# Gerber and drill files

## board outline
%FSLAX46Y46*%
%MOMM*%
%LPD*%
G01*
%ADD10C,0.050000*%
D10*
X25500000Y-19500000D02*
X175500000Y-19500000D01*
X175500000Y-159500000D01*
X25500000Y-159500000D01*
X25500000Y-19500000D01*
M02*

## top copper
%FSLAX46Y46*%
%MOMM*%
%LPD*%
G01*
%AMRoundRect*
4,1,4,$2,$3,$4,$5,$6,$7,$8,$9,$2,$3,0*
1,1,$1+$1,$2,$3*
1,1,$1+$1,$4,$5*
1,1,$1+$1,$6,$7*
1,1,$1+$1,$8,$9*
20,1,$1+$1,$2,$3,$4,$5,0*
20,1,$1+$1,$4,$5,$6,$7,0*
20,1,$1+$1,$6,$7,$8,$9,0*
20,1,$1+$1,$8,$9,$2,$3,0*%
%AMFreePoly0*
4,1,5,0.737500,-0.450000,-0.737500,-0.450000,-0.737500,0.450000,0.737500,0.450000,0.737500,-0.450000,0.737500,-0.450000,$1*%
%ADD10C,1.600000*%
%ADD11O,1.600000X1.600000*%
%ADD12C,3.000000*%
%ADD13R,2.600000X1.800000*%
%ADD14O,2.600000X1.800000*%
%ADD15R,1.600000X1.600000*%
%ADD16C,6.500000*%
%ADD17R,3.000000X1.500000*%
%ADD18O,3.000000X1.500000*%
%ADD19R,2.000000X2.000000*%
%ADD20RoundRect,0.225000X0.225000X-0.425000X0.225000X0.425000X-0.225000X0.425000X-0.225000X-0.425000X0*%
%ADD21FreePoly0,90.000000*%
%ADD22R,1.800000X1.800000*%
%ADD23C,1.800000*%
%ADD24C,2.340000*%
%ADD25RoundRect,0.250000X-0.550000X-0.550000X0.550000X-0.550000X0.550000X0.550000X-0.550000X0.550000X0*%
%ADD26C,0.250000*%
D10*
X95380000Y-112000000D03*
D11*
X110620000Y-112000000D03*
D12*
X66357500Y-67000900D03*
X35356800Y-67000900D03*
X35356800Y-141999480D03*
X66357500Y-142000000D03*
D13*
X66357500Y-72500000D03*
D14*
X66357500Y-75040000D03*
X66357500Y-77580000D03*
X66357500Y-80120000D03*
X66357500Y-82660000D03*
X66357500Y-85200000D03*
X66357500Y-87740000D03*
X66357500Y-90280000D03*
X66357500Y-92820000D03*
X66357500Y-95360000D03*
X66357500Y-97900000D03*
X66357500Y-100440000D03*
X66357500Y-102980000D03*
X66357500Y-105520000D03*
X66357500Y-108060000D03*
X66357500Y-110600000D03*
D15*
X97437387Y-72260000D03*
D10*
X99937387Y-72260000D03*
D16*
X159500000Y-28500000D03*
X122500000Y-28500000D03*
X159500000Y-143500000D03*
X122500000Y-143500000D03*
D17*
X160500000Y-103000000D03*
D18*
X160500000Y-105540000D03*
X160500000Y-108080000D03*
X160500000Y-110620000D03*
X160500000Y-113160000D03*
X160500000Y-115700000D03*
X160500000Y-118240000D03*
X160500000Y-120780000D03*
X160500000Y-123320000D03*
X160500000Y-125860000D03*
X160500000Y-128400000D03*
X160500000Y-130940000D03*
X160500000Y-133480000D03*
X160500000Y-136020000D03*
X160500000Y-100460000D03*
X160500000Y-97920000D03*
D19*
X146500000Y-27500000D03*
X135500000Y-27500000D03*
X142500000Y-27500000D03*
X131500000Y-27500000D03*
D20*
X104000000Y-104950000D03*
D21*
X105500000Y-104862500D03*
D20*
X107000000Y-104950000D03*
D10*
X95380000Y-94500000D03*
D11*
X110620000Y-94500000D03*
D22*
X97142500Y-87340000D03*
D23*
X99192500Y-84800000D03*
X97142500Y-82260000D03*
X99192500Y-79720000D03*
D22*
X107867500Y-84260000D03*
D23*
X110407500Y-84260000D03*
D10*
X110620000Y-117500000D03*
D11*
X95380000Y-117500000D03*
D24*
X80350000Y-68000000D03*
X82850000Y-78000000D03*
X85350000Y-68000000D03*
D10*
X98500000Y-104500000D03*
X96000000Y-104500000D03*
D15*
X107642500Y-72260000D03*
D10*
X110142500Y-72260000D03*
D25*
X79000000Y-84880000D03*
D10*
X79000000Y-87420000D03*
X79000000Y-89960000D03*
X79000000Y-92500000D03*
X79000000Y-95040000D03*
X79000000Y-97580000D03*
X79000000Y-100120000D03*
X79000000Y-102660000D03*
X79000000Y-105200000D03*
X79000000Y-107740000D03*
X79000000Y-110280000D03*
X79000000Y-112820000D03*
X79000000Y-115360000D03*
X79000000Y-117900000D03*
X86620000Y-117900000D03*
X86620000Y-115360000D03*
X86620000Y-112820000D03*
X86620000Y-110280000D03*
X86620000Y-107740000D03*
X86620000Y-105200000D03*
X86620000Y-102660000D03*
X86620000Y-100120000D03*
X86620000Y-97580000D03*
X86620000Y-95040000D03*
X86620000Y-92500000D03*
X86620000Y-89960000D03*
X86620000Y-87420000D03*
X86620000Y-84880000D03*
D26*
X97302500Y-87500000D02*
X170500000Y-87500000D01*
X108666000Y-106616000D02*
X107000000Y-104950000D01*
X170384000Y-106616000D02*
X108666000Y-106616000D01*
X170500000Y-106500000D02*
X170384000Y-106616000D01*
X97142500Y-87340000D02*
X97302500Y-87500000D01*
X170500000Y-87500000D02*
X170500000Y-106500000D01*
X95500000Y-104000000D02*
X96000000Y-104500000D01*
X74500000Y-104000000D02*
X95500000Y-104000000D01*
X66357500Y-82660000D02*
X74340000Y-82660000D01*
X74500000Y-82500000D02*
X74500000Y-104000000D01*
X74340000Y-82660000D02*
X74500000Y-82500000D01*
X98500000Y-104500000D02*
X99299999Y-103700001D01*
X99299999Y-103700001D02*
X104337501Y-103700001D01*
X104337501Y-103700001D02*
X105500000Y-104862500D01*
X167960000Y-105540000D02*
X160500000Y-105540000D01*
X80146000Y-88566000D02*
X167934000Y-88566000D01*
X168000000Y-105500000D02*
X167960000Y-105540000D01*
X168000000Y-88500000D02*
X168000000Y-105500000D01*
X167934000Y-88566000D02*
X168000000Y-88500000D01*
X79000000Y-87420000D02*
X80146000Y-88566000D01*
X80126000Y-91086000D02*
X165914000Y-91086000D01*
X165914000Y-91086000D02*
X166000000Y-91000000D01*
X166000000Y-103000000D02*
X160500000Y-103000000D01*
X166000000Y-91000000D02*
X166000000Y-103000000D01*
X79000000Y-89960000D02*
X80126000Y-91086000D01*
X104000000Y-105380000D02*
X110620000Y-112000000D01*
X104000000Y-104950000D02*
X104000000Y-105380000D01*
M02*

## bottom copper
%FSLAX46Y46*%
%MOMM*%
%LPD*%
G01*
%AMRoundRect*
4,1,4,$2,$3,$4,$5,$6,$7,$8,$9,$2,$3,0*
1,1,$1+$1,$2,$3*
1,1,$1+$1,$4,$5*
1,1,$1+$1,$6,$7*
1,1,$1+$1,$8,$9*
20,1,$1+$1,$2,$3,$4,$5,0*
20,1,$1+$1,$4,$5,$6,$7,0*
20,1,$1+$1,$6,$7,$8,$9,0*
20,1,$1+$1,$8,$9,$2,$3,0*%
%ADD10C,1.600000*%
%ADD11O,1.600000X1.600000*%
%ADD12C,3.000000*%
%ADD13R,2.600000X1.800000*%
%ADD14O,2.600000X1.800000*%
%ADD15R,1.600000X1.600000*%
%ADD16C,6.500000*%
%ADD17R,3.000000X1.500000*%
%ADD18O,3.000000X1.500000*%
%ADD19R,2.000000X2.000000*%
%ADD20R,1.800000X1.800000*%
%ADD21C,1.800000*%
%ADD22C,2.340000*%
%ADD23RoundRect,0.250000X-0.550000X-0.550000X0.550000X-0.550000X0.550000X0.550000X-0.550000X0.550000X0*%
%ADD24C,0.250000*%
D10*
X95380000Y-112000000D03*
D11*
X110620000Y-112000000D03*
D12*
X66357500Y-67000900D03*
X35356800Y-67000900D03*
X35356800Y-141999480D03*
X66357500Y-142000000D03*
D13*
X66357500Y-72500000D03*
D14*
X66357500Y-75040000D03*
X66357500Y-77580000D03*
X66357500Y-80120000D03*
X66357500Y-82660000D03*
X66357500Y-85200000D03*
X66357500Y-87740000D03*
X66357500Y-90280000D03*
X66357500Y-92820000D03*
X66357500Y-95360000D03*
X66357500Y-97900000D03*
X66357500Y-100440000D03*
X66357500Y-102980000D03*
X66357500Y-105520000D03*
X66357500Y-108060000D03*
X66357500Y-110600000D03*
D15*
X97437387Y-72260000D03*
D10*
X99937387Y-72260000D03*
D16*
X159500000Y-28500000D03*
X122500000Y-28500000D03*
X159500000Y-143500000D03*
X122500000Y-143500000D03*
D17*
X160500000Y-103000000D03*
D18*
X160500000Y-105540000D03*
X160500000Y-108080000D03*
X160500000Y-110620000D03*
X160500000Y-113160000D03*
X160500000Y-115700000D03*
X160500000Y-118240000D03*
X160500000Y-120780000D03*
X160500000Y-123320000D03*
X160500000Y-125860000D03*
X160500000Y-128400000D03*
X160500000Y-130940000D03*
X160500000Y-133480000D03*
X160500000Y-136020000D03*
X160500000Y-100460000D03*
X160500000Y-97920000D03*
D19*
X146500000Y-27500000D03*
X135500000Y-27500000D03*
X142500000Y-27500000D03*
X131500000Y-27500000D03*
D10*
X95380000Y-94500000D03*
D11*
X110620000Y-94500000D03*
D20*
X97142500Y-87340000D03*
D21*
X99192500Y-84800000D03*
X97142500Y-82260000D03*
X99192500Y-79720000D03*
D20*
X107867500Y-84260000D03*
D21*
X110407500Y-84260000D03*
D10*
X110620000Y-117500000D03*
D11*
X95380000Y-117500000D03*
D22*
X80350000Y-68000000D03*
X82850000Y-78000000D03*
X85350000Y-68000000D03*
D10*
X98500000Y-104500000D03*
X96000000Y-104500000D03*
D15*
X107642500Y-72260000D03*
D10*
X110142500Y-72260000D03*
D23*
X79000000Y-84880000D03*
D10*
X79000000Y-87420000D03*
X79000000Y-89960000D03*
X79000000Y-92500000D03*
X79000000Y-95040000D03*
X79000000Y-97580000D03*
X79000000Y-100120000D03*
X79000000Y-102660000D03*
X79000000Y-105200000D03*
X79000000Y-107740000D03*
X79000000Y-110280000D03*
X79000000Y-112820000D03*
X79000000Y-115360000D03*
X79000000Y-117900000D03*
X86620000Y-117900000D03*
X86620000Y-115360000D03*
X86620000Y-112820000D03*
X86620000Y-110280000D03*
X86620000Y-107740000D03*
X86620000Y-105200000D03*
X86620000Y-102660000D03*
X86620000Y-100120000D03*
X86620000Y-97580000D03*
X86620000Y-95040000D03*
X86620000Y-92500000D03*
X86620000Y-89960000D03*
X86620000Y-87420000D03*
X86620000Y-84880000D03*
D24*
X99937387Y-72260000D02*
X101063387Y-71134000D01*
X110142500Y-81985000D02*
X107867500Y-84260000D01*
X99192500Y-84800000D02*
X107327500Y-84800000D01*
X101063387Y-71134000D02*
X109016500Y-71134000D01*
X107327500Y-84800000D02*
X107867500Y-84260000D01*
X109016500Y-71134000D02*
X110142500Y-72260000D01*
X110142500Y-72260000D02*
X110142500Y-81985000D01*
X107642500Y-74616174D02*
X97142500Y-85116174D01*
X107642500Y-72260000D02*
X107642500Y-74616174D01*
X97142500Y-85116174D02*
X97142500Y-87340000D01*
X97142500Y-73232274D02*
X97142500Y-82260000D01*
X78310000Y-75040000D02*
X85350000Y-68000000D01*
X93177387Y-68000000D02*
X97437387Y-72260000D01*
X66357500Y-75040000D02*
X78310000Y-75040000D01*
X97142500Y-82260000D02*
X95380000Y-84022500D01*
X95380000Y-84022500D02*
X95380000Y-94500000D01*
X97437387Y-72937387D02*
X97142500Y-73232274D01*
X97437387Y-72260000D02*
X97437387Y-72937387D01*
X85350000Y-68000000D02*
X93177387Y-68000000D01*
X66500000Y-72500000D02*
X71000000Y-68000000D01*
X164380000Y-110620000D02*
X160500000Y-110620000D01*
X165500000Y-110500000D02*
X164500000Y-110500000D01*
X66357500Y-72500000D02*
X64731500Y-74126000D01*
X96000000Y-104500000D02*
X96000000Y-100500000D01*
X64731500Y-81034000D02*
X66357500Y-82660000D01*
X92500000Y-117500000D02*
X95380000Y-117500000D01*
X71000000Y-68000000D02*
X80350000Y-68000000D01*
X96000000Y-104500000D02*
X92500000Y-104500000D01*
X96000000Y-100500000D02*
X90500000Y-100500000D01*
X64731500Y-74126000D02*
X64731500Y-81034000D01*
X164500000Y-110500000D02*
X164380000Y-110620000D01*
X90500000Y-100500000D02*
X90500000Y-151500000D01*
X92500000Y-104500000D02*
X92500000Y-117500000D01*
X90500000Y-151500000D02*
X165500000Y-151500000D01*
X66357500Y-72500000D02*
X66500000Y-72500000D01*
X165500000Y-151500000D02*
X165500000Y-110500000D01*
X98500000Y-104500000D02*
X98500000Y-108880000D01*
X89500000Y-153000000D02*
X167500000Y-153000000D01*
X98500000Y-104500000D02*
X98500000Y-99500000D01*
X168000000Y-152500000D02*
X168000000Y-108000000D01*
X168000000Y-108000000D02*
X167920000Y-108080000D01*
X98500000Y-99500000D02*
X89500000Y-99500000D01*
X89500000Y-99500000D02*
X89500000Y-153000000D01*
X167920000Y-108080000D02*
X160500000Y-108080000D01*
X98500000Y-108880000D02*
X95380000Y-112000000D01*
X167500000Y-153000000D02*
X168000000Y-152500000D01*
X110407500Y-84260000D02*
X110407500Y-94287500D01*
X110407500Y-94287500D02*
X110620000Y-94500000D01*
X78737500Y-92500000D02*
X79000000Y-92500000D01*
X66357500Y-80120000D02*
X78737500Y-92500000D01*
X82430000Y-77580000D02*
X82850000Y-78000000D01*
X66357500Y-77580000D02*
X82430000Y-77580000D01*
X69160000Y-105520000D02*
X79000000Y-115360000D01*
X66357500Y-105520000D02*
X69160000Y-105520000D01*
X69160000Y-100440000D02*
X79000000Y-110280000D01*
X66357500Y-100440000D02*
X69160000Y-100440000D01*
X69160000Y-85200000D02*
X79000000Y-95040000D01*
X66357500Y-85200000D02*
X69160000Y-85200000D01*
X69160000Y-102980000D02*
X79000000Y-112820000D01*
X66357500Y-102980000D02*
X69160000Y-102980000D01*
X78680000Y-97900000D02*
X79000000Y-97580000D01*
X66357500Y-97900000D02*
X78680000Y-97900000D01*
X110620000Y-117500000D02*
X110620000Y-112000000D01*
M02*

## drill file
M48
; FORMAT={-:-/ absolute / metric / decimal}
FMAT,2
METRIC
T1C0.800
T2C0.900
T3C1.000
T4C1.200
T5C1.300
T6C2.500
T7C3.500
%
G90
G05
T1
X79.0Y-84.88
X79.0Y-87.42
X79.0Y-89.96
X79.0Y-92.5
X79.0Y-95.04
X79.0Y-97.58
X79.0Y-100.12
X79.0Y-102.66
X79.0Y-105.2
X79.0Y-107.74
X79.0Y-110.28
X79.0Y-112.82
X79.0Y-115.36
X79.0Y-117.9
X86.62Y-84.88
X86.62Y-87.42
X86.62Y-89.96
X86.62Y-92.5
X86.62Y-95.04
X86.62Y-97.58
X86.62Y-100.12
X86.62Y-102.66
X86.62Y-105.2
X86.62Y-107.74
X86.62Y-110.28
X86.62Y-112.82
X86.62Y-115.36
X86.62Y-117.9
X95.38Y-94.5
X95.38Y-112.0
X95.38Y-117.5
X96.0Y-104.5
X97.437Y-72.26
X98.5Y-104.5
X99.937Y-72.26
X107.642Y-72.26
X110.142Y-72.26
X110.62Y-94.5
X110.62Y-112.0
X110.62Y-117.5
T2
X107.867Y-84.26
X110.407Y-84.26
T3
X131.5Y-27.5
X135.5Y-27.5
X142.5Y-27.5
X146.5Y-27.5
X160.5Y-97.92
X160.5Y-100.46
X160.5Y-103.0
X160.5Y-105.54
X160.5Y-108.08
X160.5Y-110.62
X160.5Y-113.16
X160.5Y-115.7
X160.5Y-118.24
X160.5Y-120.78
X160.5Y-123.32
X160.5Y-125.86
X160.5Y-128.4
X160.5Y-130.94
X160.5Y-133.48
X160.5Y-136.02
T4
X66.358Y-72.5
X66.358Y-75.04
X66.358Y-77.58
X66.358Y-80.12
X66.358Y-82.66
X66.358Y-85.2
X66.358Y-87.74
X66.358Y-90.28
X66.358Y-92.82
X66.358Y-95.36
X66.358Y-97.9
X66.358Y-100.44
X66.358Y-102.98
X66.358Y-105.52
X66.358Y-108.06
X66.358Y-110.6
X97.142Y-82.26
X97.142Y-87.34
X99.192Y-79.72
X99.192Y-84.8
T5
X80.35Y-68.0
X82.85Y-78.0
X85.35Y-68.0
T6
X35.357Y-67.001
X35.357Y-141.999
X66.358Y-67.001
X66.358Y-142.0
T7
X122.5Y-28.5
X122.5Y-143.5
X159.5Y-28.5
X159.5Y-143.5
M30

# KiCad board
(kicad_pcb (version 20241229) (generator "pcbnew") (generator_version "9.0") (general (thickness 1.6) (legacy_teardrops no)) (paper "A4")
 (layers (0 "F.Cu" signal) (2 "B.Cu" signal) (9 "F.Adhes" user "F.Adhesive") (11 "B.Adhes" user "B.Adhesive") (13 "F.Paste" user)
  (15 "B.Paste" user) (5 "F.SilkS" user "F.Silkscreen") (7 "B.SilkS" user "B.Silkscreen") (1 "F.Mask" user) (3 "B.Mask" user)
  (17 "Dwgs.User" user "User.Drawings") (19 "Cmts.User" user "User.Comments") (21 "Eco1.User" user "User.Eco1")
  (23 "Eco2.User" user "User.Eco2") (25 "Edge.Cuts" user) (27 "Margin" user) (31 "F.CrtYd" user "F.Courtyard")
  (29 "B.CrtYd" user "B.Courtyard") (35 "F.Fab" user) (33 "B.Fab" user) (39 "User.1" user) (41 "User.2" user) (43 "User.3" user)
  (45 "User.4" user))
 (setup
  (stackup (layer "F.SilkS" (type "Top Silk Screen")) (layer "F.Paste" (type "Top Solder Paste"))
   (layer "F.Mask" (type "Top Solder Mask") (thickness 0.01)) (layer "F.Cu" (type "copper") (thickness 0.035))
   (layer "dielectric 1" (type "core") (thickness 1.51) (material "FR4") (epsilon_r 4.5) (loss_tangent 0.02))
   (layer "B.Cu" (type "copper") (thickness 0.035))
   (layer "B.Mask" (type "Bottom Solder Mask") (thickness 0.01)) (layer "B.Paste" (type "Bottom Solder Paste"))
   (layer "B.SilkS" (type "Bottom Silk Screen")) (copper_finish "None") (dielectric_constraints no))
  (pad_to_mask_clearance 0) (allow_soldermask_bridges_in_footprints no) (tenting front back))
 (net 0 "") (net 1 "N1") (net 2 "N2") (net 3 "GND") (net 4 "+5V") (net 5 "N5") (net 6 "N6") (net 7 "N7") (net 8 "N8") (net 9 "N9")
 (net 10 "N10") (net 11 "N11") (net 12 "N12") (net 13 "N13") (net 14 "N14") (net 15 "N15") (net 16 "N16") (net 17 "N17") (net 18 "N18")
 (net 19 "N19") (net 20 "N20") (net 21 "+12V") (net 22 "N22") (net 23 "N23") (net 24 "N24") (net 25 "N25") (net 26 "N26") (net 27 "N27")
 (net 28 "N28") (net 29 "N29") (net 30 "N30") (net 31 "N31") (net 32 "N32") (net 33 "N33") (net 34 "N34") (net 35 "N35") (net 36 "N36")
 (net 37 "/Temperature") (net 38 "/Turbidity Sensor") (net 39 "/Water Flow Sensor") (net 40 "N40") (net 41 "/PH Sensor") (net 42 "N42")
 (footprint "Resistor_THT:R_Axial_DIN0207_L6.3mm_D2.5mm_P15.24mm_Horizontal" (layer "F.Cu") (at 95.38 112)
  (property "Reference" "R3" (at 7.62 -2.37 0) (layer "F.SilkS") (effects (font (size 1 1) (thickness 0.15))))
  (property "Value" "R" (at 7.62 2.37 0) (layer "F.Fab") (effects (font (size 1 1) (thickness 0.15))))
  (pad "1" thru_hole circle (at 0 0) (size 1.6 1.6) (drill 0.8) (layers "*.Cu" "*.Mask") (remove_unused_layers no) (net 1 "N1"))
  (pad "2" thru_hole oval (at 15.24 0) (size 1.6 1.6) (drill 0.8) (layers "*.Cu" "*.Mask") (remove_unused_layers no) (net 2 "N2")))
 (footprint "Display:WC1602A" (layer "F.Cu") (at 66.3575 72.5 -90)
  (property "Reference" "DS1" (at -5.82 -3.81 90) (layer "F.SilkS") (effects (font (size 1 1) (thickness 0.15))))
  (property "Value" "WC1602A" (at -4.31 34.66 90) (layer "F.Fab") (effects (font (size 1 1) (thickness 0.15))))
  (pad "" thru_hole circle (at -5.4991 0 270) (size 3 3) (drill 2.5) (layers "*.Cu" "*.Mask") (remove_unused_layers no))
  (pad "" thru_hole circle (at -5.4991 31.0007 270) (size 3 3) (drill 2.5) (layers "*.Cu" "*.Mask") (remove_unused_layers no))
  (pad "" thru_hole circle (at 69.49948 31.0007 270) (size 3 3) (drill 2.5) (layers "*.Cu" "*.Mask") (remove_unused_layers no))
  (pad "" thru_hole circle (at 69.5 0 270) (size 3 3) (drill 2.5) (layers "*.Cu" "*.Mask") (remove_unused_layers no))
  (pad "1" thru_hole rect (at 0 0 270) (size 1.8 2.6) (drill 1.2) (layers "*.Cu" "*.Mask") (remove_unused_layers no) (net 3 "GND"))
  (pad "2" thru_hole oval (at 2.54 0 270) (size 1.8 2.6) (drill 1.2) (layers "*.Cu" "*.Mask") (remove_unused_layers no) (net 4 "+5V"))
  (pad "3" thru_hole oval (at 5.08 0 270) (size 1.8 2.6) (drill 1.2) (layers "*.Cu" "*.Mask") (remove_unused_layers no) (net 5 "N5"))
  (pad "4" thru_hole oval (at 7.62 0 270) (size 1.8 2.6) (drill 1.2) (layers "*.Cu" "*.Mask") (remove_unused_layers no) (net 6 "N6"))
  (pad "5" thru_hole oval (at 10.16 0 270) (size 1.8 2.6) (drill 1.2) (layers "*.Cu" "*.Mask") (remove_unused_layers no) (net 3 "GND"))
  (pad "6" thru_hole oval (at 12.7 0 270) (size 1.8 2.6) (drill 1.2) (layers "*.Cu" "*.Mask") (remove_unused_layers no) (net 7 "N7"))
  (pad "7" thru_hole oval (at 15.24 0 270) (size 1.8 2.6) (drill 1.2) (layers "*.Cu" "*.Mask") (remove_unused_layers no) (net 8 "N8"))
  (pad "8" thru_hole oval (at 17.78 0 270) (size 1.8 2.6) (drill 1.2) (layers "*.Cu" "*.Mask") (remove_unused_layers no) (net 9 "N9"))
  (pad "9" thru_hole oval (at 20.32 0 270) (size 1.8 2.6) (drill 1.2) (layers "*.Cu" "*.Mask") (remove_unused_layers no) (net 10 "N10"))
  (pad "10" thru_hole oval (at 22.86 0 270) (size 1.8 2.6) (drill 1.2) (layers "*.Cu" "*.Mask") (remove_unused_layers no) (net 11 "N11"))
  (pad "11" thru_hole oval (at 25.4 0 270) (size 1.8 2.6) (drill 1.2) (layers "*.Cu" "*.Mask") (remove_unused_layers no) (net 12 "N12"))
  (pad "12" thru_hole oval (at 27.94 0 270) (size 1.8 2.6) (drill 1.2) (layers "*.Cu" "*.Mask") (remove_unused_layers no) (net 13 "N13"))
  (pad "13" thru_hole oval (at 30.48 0 270) (size 1.8 2.6) (drill 1.2) (layers "*.Cu" "*.Mask") (remove_unused_layers no) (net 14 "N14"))
  (pad "14" thru_hole oval (at 33.02 0 270) (size 1.8 2.6) (drill 1.2) (layers "*.Cu" "*.Mask") (remove_unused_layers no) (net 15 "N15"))
  (pad "15" thru_hole oval (at 35.56 0 270) (size 1.8 2.6) (drill 1.2) (layers "*.Cu" "*.Mask") (remove_unused_layers no) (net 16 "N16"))
  (pad "16" thru_hole oval (at 38.1 0 270) (size 1.8 2.6) (drill 1.2) (layers "*.Cu" "*.Mask") (remove_unused_layers no) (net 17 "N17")))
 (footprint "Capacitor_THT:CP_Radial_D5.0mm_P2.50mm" (layer "F.Cu") (at 97.437387 72.26)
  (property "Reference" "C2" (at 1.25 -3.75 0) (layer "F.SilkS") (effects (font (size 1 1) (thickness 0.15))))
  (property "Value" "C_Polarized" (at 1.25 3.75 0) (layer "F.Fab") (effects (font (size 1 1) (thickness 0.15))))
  (pad "1" thru_hole rect (at 0 0) (size 1.6 1.6) (drill 0.8) (layers "*.Cu" "*.Mask") (remove_unused_layers no) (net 4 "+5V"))
  (pad "2" thru_hole circle (at 2.5 0) (size 1.6 1.6) (drill 0.8) (layers "*.Cu" "*.Mask") (remove_unused_layers no) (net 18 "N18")))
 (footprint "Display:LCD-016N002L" (layer "F.Cu") (at 160.5 103 -90)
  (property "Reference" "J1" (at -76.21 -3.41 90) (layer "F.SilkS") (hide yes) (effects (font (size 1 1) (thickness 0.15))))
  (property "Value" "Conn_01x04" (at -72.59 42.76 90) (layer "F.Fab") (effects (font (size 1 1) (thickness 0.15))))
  (pad "" thru_hole circle (at -74.5 1 90) (size 6.5 6.5) (drill 3.5) (layers "*.Cu" "*.Mask") (remove_unused_layers no))
  (pad "" thru_hole circle (at -74.5 38 90) (size 6.5 6.5) (drill 3.5) (layers "*.Cu" "*.Mask") (remove_unused_layers no))
  (pad "" thru_hole circle (at 40.5 1 90) (size 6.5 6.5) (drill 3.5) (layers "*.Cu" "*.Mask") (remove_unused_layers no))
  (pad "" thru_hole circle (at 40.5 38 90) (size 6.5 6.5) (drill 3.5) (layers "*.Cu" "*.Mask") (remove_unused_layers no))
  (pad "1" thru_hole rect (at 0 0 90) (size 1.5 3) (drill 1) (layers "*.Cu" "*.Mask") (remove_unused_layers no) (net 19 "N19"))
  (pad "2" thru_hole oval (at 2.54 0 90) (size 1.5 3) (drill 1) (layers "*.Cu" "*.Mask") (remove_unused_layers no) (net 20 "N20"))
  (pad "3" thru_hole oval (at 5.08 0 90) (size 1.5 3) (drill 1) (layers "*.Cu" "*.Mask") (remove_unused_layers no) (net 1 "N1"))
  (pad "4" thru_hole oval (at 7.62 0 90) (size 1.5 3) (drill 1) (layers "*.Cu" "*.Mask") (remove_unused_layers no) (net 3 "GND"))
  (pad "5" thru_hole oval (at 10.16 0 90) (size 1.5 3) (drill 1) (layers "*.Cu" "*.Mask") (remove_unused_layers no))
  (pad "6" thru_hole oval (at 12.7 0 90) (size 1.5 3) (drill 1) (layers "*.Cu" "*.Mask") (remove_unused_layers no))
  (pad "7" thru_hole oval (at 15.24 0 90) (size 1.5 3) (drill 1) (layers "*.Cu" "*.Mask") (remove_unused_layers no))
  (pad "8" thru_hole oval (at 17.78 0 90) (size 1.5 3) (drill 1) (layers "*.Cu" "*.Mask") (remove_unused_layers no))
  (pad "9" thru_hole oval (at 20.32 0 90) (size 1.5 3) (drill 1) (layers "*.Cu" "*.Mask") (remove_unused_layers no))
  (pad "10" thru_hole oval (at 22.86 0 90) (size 1.5 3) (drill 1) (layers "*.Cu" "*.Mask") (remove_unused_layers no))
  (pad "11" thru_hole oval (at 25.4 0 90) (size 1.5 3) (drill 1) (layers "*.Cu" "*.Mask") (remove_unused_layers no))
  (pad "12" thru_hole oval (at 27.94 0 90) (size 1.5 3) (drill 1) (layers "*.Cu" "*.Mask") (remove_unused_layers no))
  (pad "13" thru_hole oval (at 30.48 0 90) (size 1.5 3) (drill 1) (layers "*.Cu" "*.Mask") (remove_unused_layers no))
  (pad "14" thru_hole oval (at 33.02 0 90) (size 1.5 3) (drill 1) (layers "*.Cu" "*.Mask") (remove_unused_layers no))
  (pad "15" thru_hole oval (at -2.54 0 90) (size 1.5 3) (drill 1) (layers "*.Cu" "*.Mask") (remove_unused_layers no))
  (pad "16" thru_hole oval (at -5.08 0 90) (size 1.5 3) (drill 1) (layers "*.Cu" "*.Mask") (remove_unused_layers no))
  (pad "A1" thru_hole rect (at -75.5 14 90) (size 2 2) (drill 1) (layers "*.Cu" "*.Mask") (remove_unused_layers no))
  (pad "A2" thru_hole rect (at -75.5 25 90) (size 2 2) (drill 1) (layers "*.Cu" "*.Mask") (remove_unused_layers no))
  (pad "K1" thru_hole rect (at -75.5 18 90) (size 2 2) (drill 1) (layers "*.Cu" "*.Mask") (remove_unused_layers no))
  (pad "K2" thru_hole rect (at -75.5 29 90) (size 2 2) (drill 1) (layers "*.Cu" "*.Mask") (remove_unused_layers no)))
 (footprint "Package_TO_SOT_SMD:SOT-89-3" (layer "F.Cu") (at 105.5 103 90)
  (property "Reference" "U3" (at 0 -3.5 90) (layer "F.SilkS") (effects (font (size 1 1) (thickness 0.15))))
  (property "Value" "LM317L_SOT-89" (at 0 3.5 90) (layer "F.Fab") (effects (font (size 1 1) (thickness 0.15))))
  (pad "1" smd roundrect (at -1.95 -1.5 90) (size 1.3 0.9) (layers "F.Cu" "F.Mask" "F.Paste") (roundrect_rratio 0.25) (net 2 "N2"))
  (pad "2" smd custom (at -1.8625 0 90) (size 1.475 0.9) (layers "F.Cu" "F.Mask" "F.Paste") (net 1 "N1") (zone_connect 2)
   (thermal_bridge_angle 45) (options (clearance outline) (anchor rect)) (primitives))
  (pad "3" smd roundrect (at -1.95 1.5 90) (size 1.3 0.9) (layers "F.Cu" "F.Mask" "F.Paste") (roundrect_rratio 0.25) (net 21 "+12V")))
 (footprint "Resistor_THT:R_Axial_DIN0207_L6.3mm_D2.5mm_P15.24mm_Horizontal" (layer "F.Cu") (at 95.38 94.5)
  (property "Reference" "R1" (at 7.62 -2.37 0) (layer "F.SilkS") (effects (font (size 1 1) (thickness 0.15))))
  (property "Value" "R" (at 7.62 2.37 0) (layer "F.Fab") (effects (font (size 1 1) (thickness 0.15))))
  (pad "1" thru_hole circle (at 0 0) (size 1.6 1.6) (drill 0.8) (layers "*.Cu" "*.Mask") (remove_unused_layers no) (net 4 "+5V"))
  (pad "2" thru_hole oval (at 15.24 0) (size 1.6 1.6) (drill 0.8) (layers "*.Cu" "*.Mask") (remove_unused_layers no) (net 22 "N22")))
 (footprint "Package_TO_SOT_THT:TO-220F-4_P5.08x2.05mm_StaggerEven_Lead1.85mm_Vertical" (layer "F.Cu") (at 97.1425 87.34 90)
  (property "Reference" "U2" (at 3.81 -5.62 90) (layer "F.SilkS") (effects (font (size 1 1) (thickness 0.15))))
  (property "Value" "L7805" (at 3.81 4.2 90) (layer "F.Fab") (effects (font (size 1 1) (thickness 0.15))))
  (pad "1" thru_hole rect (at 0 0 90) (size 1.8 1.8) (drill 1.2) (layers "*.Cu" "*.Mask") (remove_unused_layers no) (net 21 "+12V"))
  (pad "2" thru_hole circle (at 2.54 2.05 90) (size 1.8 1.8) (drill 1.2) (layers "*.Cu" "*.Mask") (remove_unused_layers no) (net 18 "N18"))
  (pad "3" thru_hole circle (at 5.08 0 90) (size 1.8 1.8) (drill 1.2) (layers "*.Cu" "*.Mask") (remove_unused_layers no) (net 4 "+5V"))
  (pad "4" thru_hole circle (at 7.62 2.05 90) (size 1.8 1.8) (drill 1.2) (layers "*.Cu" "*.Mask") (remove_unused_layers no)))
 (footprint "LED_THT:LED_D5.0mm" (layer "F.Cu") (at 107.8675 84.26)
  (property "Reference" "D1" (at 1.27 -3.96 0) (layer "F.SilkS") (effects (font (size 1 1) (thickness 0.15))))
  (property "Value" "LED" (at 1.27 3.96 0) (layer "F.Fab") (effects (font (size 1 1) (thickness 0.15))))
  (pad "1" thru_hole rect (at 0 0) (size 1.8 1.8) (drill 0.9) (layers "*.Cu" "*.Mask") (remove_unused_layers no) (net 18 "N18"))
  (pad "2" thru_hole circle (at 2.54 0) (size 1.8 1.8) (drill 0.9) (layers "*.Cu" "*.Mask") (remove_unused_layers no) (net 22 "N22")))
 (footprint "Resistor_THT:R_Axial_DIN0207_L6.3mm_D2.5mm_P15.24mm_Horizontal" (layer "F.Cu") (at 110.62 117.5 180)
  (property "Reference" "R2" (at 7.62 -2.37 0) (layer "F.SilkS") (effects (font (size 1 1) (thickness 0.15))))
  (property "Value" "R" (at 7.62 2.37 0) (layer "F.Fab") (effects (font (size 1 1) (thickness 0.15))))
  (pad "1" thru_hole circle (at 0 0 180) (size 1.6 1.6) (drill 0.8) (layers "*.Cu" "*.Mask") (remove_unused_layers no) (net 2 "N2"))
  (pad "2" thru_hole oval (at 15.24 0 180) (size 1.6 1.6) (drill 0.8) (layers "*.Cu" "*.Mask") (remove_unused_layers no) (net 3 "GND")))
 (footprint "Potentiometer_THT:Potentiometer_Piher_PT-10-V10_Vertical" (layer "F.Cu") (at 80.35 68 -90)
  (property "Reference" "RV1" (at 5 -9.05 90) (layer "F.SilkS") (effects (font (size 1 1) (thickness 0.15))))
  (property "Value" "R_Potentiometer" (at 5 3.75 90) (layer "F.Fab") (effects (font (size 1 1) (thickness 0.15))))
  (pad "1" thru_hole circle (at 0 0 270) (size 2.34 2.34) (drill 1.3) (layers "*.Cu" "*.Mask") (remove_unused_layers no) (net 3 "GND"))
  (pad "2" thru_hole circle (at 10 -2.5 270) (size 2.34 2.34) (drill 1.3) (layers "*.Cu" "*.Mask") (remove_unused_layers no) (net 5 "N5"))
  (pad "3" thru_hole circle (at 0 -5 270) (size 2.34 2.34) (drill 1.3) (layers "*.Cu" "*.Mask") (remove_unused_layers no) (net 4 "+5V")))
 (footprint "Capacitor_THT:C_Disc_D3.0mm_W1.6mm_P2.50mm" (layer "F.Cu") (at 98.5 104.5 180)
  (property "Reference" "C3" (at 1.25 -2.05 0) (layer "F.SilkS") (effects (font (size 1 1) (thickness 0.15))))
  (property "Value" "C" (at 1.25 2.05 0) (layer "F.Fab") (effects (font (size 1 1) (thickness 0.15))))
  (pad "1" thru_hole circle (at 0 0 180) (size 1.6 1.6) (drill 0.8) (layers "*.Cu" "*.Mask") (remove_unused_layers no) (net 1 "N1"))
  (pad "2" thru_hole circle (at 2.5 0 180) (size 1.6 1.6) (drill 0.8) (layers "*.Cu" "*.Mask") (remove_unused_layers no) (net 3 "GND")))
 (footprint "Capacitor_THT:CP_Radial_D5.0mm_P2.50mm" (layer "F.Cu") (at 107.6425 72.26)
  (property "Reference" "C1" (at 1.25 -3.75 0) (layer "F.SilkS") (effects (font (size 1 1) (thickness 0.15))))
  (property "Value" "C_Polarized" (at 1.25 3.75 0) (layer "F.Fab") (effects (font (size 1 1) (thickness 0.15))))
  (pad "1" thru_hole rect (at 0 0) (size 1.6 1.6) (drill 0.8) (layers "*.Cu" "*.Mask") (remove_unused_layers no) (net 21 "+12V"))
  (pad "2" thru_hole circle (at 2.5 0) (size 1.6 1.6) (drill 0.8) (layers "*.Cu" "*.Mask") (remove_unused_layers no) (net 18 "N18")))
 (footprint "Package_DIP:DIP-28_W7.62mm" (layer "F.Cu") (at 79 84.88)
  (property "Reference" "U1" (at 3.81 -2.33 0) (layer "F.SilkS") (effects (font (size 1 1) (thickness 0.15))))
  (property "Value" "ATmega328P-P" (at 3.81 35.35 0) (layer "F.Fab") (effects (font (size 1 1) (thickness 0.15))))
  (pad "1" thru_hole roundrect (at 0 0) (size 1.6 1.6) (drill 0.8) (layers "*.Cu" "*.Mask") (remove_unused_layers no)
   (roundrect_rratio 0.15625) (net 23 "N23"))
  (pad "2" thru_hole circle (at 0 2.54) (size 1.6 1.6) (drill 0.8) (layers "*.Cu" "*.Mask") (remove_unused_layers no) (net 20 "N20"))
  (pad "3" thru_hole circle (at 0 5.08) (size 1.6 1.6) (drill 0.8) (layers "*.Cu" "*.Mask") (remove_unused_layers no) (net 19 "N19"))
  (pad "4" thru_hole circle (at 0 7.62) (size 1.6 1.6) (drill 0.8) (layers "*.Cu" "*.Mask") (remove_unused_layers no) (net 6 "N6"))
  (pad "5" thru_hole circle (at 0 10.16) (size 1.6 1.6) (drill 0.8) (layers "*.Cu" "*.Mask") (remove_unused_layers no) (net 7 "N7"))
  (pad "6" thru_hole circle (at 0 12.7) (size 1.6 1.6) (drill 0.8) (layers "*.Cu" "*.Mask") (remove_unused_layers no) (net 12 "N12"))
  (pad "7" thru_hole circle (at 0 15.24) (size 1.6 1.6) (drill 0.8) (layers "*.Cu" "*.Mask") (remove_unused_layers no) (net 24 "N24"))
  (pad "8" thru_hole circle (at 0 17.78) (size 1.6 1.6) (drill 0.8) (layers "*.Cu" "*.Mask") (remove_unused_layers no) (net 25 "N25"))
  (pad "9" thru_hole circle (at 0 20.32) (size 1.6 1.6) (drill 0.8) (layers "*.Cu" "*.Mask") (remove_unused_layers no) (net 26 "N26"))
  (pad "10" thru_hole circle (at 0 22.86) (size 1.6 1.6) (drill 0.8) (layers "*.Cu" "*.Mask") (remove_unused_layers no) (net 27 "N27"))
  (pad "11" thru_hole circle (at 0 25.4) (size 1.6 1.6) (drill 0.8) (layers "*.Cu" "*.Mask") (remove_unused_layers no) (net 13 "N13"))
  (pad "12" thru_hole circle (at 0 27.94) (size 1.6 1.6) (drill 0.8) (layers "*.Cu" "*.Mask") (remove_unused_layers no) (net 14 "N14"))
  (pad "13" thru_hole circle (at 0 30.48) (size 1.6 1.6) (drill 0.8) (layers "*.Cu" "*.Mask") (remove_unused_layers no) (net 15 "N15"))
  (pad "14" thru_hole circle (at 0 33.02) (size 1.6 1.6) (drill 0.8) (layers "*.Cu" "*.Mask") (remove_unused_layers no) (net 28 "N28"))
  (pad "15" thru_hole circle (at 7.62 33.02) (size 1.6 1.6) (drill 0.8) (layers "*.Cu" "*.Mask") (remove_unused_layers no) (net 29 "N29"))
  (pad "16" thru_hole circle (at 7.62 30.48) (size 1.6 1.6) (drill 0.8) (layers "*.Cu" "*.Mask") (remove_unused_layers no) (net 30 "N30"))
  (pad "17" thru_hole circle (at 7.62 27.94) (size 1.6 1.6) (drill 0.8) (layers "*.Cu" "*.Mask") (remove_unused_layers no) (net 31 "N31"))
  (pad "18" thru_hole circle (at 7.62 25.4) (size 1.6 1.6) (drill 0.8) (layers "*.Cu" "*.Mask") (remove_unused_layers no) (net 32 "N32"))
  (pad "19" thru_hole circle (at 7.62 22.86) (size 1.6 1.6) (drill 0.8) (layers "*.Cu" "*.Mask") (remove_unused_layers no) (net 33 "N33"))
  (pad "20" thru_hole circle (at 7.62 20.32) (size 1.6 1.6) (drill 0.8) (layers "*.Cu" "*.Mask") (remove_unused_layers no) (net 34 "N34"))
  (pad "21" thru_hole circle (at 7.62 17.78) (size 1.6 1.6) (drill 0.8) (layers "*.Cu" "*.Mask") (remove_unused_layers no) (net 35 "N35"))
  (pad "22" thru_hole circle (at 7.62 15.24) (size 1.6 1.6) (drill 0.8) (layers "*.Cu" "*.Mask") (remove_unused_layers no) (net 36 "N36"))
  (pad "23" thru_hole circle (at 7.62 12.7) (size 1.6 1.6) (drill 0.8) (layers "*.Cu" "*.Mask") (remove_unused_layers no)
   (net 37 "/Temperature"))
  (pad "24" thru_hole circle (at 7.62 10.16) (size 1.6 1.6) (drill 0.8) (layers "*.Cu" "*.Mask") (remove_unused_layers no)
   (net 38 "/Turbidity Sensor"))
  (pad "25" thru_hole circle (at 7.62 7.62) (size 1.6 1.6) (drill 0.8) (layers "*.Cu" "*.Mask") (remove_unused_layers no)
   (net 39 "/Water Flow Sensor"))
  (pad "26" thru_hole circle (at 7.62 5.08) (size 1.6 1.6) (drill 0.8) (layers "*.Cu" "*.Mask") (remove_unused_layers no) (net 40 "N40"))
  (pad "27" thru_hole circle (at 7.62 2.54) (size 1.6 1.6) (drill 0.8) (layers "*.Cu" "*.Mask") (remove_unused_layers no)
   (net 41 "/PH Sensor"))
  (pad "28" thru_hole circle (at 7.62 0) (size 1.6 1.6) (drill 0.8) (layers "*.Cu" "*.Mask") (remove_unused_layers no) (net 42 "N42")))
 (gr_rect (start 25.5 19.5) (end 175.5 159.5) (stroke (width 0.05) (type default)) (fill no) (layer "Edge.Cuts"))
 (segment (start 99.937387 72.26) (end 101.063387 71.134) (width 0.25) (layer "B.Cu") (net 18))
 (segment (start 110.1425 81.985) (end 107.8675 84.26) (width 0.25) (layer "B.Cu") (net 18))
 (segment (start 99.1925 84.8) (end 107.3275 84.8) (width 0.25) (layer "B.Cu") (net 18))
 (segment (start 101.063387 71.134) (end 109.0165 71.134) (width 0.25) (layer "B.Cu") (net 18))
 (segment (start 107.3275 84.8) (end 107.8675 84.26) (width 0.25) (layer "B.Cu") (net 18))
 (segment (start 109.0165 71.134) (end 110.1425 72.26) (width 0.25) (layer "B.Cu") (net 18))
 (segment (start 110.1425 72.26) (end 110.1425 81.985) (width 0.25) (layer "B.Cu") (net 18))
 (segment (start 97.3025 87.5) (end 170.5 87.5) (width 0.25) (layer "F.Cu") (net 21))
 (segment (start 108.666 106.616) (end 107 104.95) (width 0.25) (layer "F.Cu") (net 21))
 (segment (start 170.384 106.616) (end 108.666 106.616) (width 0.25) (layer "F.Cu") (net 21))
 (segment (start 170.5 106.5) (end 170.384 106.616) (width 0.25) (layer "F.Cu") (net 21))
 (segment (start 97.1425 87.34) (end 97.3025 87.5) (width 0.25) (layer "F.Cu") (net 21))
 (segment (start 170.5 87.5) (end 170.5 106.5) (width 0.25) (layer "F.Cu") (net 21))
 (segment (start 107.6425 74.616174) (end 97.1425 85.116174) (width 0.25) (layer "B.Cu") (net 21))
 (segment (start 107.6425 72.26) (end 107.6425 74.616174) (width 0.25) (layer "B.Cu") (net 21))
 (segment (start 97.1425 85.116174) (end 97.1425 87.34) (width 0.25) (layer "B.Cu") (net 21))
 (segment (start 97.1425 73.232274) (end 97.1425 82.26) (width 0.25) (layer "B.Cu") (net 4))
 (segment (start 78.31 75.04) (end 85.35 68) (width 0.25) (layer "B.Cu") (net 4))
 (segment (start 93.177387 68) (end 97.437387 72.26) (width 0.25) (layer "B.Cu") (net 4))
 (segment (start 66.3575 75.04) (end 78.31 75.04) (width 0.25) (layer "B.Cu") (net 4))
 (segment (start 97.1425 82.26) (end 95.38 84.0225) (width 0.25) (layer "B.Cu") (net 4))
 (segment (start 95.38 84.0225) (end 95.38 94.5) (width 0.25) (layer "B.Cu") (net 4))
 (segment (start 97.437387 72.937387) (end 97.1425 73.232274) (width 0.25) (layer "B.Cu") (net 4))
 (segment (start 97.437387 72.26) (end 97.437387 72.937387) (width 0.25) (layer "B.Cu") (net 4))
 (segment (start 85.35 68) (end 93.177387 68) (width 0.25) (layer "B.Cu") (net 4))
 (segment (start 95.5 104) (end 96 104.5) (width 0.25) (layer "F.Cu") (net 3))
 (segment (start 74.5 104) (end 95.5 104) (width 0.25) (layer "F.Cu") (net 3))
 (segment (start 66.3575 82.66) (end 74.34 82.66) (width 0.25) (layer "F.Cu") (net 3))
 (segment (start 74.5 82.5) (end 74.5 104) (width 0.25) (layer "F.Cu") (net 3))
 (segment (start 74.34 82.66) (end 74.5 82.5) (width 0.25) (layer "F.Cu") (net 3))
 (segment (start 66.5 72.5) (end 71 68) (width 0.25) (layer "B.Cu") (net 3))
 (segment (start 164.38 110.62) (end 160.5 110.62) (width 0.25) (layer "B.Cu") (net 3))
 (segment (start 165.5 110.5) (end 164.5 110.5) (width 0.25) (layer "B.Cu") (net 3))
 (segment (start 66.3575 72.5) (end 64.7315 74.126) (width 0.25) (layer "B.Cu") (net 3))
 (segment (start 96 104.5) (end 96 100.5) (width 0.25) (layer "B.Cu") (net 3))
 (segment (start 64.7315 81.034) (end 66.3575 82.66) (width 0.25) (layer "B.Cu") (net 3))
 (segment (start 92.5 117.5) (end 95.38 117.5) (width 0.25) (layer "B.Cu") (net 3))
 (segment (start 71 68) (end 80.35 68) (width 0.25) (layer "B.Cu") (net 3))
 (segment (start 96 104.5) (end 92.5 104.5) (width 0.25) (layer "B.Cu") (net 3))
 (segment (start 96 100.5) (end 90.5 100.5) (width 0.25) (layer "B.Cu") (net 3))
 (segment (start 64.7315 74.126) (end 64.7315 81.034) (width 0.25) (layer "B.Cu") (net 3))
 (segment (start 164.5 110.5) (end 164.38 110.62) (width 0.25) (layer "B.Cu") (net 3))
 (segment (start 90.5 100.5) (end 90.5 151.5) (width 0.25) (layer "B.Cu") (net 3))
 (segment (start 92.5 104.5) (end 92.5 117.5) (width 0.25) (layer "B.Cu") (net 3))
 (segment (start 90.5 151.5) (end 165.5 151.5) (width 0.25) (layer "B.Cu") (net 3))
 (segment (start 66.3575 72.5) (end 66.5 72.5) (width 0.25) (layer "B.Cu") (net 3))
 (segment (start 165.5 151.5) (end 165.5 110.5) (width 0.25) (layer "B.Cu") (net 3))
 (segment (start 98.5 104.5) (end 99.299999 103.700001) (width 0.25) (layer "F.Cu") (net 1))
 (segment (start 99.299999 103.700001) (end 104.337501 103.700001) (width 0.25) (layer "F.Cu") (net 1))
 (segment (start 104.337501 103.700001) (end 105.5 104.8625) (width 0.25) (layer "F.Cu") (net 1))
 (segment (start 98.5 104.5) (end 98.5 108.88) (width 0.25) (layer "B.Cu") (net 1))
 (segment (start 89.5 153) (end 167.5 153) (width 0.25) (layer "B.Cu") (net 1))
 (segment (start 98.5 104.5) (end 98.5 99.5) (width 0.25) (layer "B.Cu") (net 1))
 (segment (start 168 152.5) (end 168 108) (width 0.25) (layer "B.Cu") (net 1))
 (segment (start 168 108) (end 167.92 108.08) (width 0.25) (layer "B.Cu") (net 1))
 (segment (start 98.5 99.5) (end 89.5 99.5) (width 0.25) (layer "B.Cu") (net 1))
 (segment (start 89.5 99.5) (end 89.5 153) (width 0.25) (layer "B.Cu") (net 1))
 (segment (start 167.92 108.08) (end 160.5 108.08) (width 0.25) (layer "B.Cu") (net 1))
 (segment (start 98.5 108.88) (end 95.38 112) (width 0.25) (layer "B.Cu") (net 1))
 (segment (start 167.5 153) (end 168 152.5) (width 0.25) (layer "B.Cu") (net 1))
 (segment (start 110.4075 84.26) (end 110.4075 94.2875) (width 0.25) (layer "B.Cu") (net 22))
 (segment (start 110.4075 94.2875) (end 110.62 94.5) (width 0.25) (layer "B.Cu") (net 22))
 (segment (start 78.7375 92.5) (end 79 92.5) (width 0.25) (layer "B.Cu") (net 6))
 (segment (start 66.3575 80.12) (end 78.7375 92.5) (width 0.25) (layer "B.Cu") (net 6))
 (segment (start 82.43 77.58) (end 82.85 78) (width 0.25) (layer "B.Cu") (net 5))
 (segment (start 66.3575 77.58) (end 82.43 77.58) (width 0.25) (layer "B.Cu") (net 5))
 (segment (start 69.16 105.52) (end 79 115.36) (width 0.25) (layer "B.Cu") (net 15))
 (segment (start 66.3575 105.52) (end 69.16 105.52) (width 0.25) (layer "B.Cu") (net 15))
 (segment (start 69.16 100.44) (end 79 110.28) (width 0.25) (layer "B.Cu") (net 13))
 (segment (start 66.3575 100.44) (end 69.16 100.44) (width 0.25) (layer "B.Cu") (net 13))
 (segment (start 69.16 85.2) (end 79 95.04) (width 0.25) (layer "B.Cu") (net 7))
 (segment (start 66.3575 85.2) (end 69.16 85.2) (width 0.25) (layer "B.Cu") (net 7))
 (segment (start 69.16 102.98) (end 79 112.82) (width 0.25) (layer "B.Cu") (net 14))
 (segment (start 66.3575 102.98) (end 69.16 102.98) (width 0.25) (layer "B.Cu") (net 14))
 (segment (start 78.68 97.9) (end 79 97.58) (width 0.25) (layer "B.Cu") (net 12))
 (segment (start 66.3575 97.9) (end 78.68 97.9) (width 0.25) (layer "B.Cu") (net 12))
 (segment (start 167.96 105.54) (end 160.5 105.54) (width 0.25) (layer "F.Cu") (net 20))
 (segment (start 80.146 88.566) (end 167.934 88.566) (width 0.25) (layer "F.Cu") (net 20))
 (segment (start 168 105.5) (end 167.96 105.54) (width 0.25) (layer "F.Cu") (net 20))
 (segment (start 168 88.5) (end 168 105.5) (width 0.25) (layer "F.Cu") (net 20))
 (segment (start 167.934 88.566) (end 168 88.5) (width 0.25) (layer "F.Cu") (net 20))
 (segment (start 79 87.42) (end 80.146 88.566) (width 0.25) (layer "F.Cu") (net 20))
 (segment (start 80.126 91.086) (end 165.914 91.086) (width 0.25) (layer "F.Cu") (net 19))
 (segment (start 165.914 91.086) (end 166 91) (width 0.25) (layer "F.Cu") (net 19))
 (segment (start 166 103) (end 160.5 103) (width 0.25) (layer "F.Cu") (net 19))
 (segment (start 166 91) (end 166 103) (width 0.25) (layer "F.Cu") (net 19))
 (segment (start 79 89.96) (end 80.126 91.086) (width 0.25) (layer "F.Cu") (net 19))
 (segment (start 104 105.38) (end 110.62 112) (width 0.25) (layer "F.Cu") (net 2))
 (segment (start 104 104.95) (end 104 105.38) (width 0.25) (layer "F.Cu") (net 2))
 (segment (start 110.62 117.5) (end 110.62 112) (width 0.25) (layer "B.Cu") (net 2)))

